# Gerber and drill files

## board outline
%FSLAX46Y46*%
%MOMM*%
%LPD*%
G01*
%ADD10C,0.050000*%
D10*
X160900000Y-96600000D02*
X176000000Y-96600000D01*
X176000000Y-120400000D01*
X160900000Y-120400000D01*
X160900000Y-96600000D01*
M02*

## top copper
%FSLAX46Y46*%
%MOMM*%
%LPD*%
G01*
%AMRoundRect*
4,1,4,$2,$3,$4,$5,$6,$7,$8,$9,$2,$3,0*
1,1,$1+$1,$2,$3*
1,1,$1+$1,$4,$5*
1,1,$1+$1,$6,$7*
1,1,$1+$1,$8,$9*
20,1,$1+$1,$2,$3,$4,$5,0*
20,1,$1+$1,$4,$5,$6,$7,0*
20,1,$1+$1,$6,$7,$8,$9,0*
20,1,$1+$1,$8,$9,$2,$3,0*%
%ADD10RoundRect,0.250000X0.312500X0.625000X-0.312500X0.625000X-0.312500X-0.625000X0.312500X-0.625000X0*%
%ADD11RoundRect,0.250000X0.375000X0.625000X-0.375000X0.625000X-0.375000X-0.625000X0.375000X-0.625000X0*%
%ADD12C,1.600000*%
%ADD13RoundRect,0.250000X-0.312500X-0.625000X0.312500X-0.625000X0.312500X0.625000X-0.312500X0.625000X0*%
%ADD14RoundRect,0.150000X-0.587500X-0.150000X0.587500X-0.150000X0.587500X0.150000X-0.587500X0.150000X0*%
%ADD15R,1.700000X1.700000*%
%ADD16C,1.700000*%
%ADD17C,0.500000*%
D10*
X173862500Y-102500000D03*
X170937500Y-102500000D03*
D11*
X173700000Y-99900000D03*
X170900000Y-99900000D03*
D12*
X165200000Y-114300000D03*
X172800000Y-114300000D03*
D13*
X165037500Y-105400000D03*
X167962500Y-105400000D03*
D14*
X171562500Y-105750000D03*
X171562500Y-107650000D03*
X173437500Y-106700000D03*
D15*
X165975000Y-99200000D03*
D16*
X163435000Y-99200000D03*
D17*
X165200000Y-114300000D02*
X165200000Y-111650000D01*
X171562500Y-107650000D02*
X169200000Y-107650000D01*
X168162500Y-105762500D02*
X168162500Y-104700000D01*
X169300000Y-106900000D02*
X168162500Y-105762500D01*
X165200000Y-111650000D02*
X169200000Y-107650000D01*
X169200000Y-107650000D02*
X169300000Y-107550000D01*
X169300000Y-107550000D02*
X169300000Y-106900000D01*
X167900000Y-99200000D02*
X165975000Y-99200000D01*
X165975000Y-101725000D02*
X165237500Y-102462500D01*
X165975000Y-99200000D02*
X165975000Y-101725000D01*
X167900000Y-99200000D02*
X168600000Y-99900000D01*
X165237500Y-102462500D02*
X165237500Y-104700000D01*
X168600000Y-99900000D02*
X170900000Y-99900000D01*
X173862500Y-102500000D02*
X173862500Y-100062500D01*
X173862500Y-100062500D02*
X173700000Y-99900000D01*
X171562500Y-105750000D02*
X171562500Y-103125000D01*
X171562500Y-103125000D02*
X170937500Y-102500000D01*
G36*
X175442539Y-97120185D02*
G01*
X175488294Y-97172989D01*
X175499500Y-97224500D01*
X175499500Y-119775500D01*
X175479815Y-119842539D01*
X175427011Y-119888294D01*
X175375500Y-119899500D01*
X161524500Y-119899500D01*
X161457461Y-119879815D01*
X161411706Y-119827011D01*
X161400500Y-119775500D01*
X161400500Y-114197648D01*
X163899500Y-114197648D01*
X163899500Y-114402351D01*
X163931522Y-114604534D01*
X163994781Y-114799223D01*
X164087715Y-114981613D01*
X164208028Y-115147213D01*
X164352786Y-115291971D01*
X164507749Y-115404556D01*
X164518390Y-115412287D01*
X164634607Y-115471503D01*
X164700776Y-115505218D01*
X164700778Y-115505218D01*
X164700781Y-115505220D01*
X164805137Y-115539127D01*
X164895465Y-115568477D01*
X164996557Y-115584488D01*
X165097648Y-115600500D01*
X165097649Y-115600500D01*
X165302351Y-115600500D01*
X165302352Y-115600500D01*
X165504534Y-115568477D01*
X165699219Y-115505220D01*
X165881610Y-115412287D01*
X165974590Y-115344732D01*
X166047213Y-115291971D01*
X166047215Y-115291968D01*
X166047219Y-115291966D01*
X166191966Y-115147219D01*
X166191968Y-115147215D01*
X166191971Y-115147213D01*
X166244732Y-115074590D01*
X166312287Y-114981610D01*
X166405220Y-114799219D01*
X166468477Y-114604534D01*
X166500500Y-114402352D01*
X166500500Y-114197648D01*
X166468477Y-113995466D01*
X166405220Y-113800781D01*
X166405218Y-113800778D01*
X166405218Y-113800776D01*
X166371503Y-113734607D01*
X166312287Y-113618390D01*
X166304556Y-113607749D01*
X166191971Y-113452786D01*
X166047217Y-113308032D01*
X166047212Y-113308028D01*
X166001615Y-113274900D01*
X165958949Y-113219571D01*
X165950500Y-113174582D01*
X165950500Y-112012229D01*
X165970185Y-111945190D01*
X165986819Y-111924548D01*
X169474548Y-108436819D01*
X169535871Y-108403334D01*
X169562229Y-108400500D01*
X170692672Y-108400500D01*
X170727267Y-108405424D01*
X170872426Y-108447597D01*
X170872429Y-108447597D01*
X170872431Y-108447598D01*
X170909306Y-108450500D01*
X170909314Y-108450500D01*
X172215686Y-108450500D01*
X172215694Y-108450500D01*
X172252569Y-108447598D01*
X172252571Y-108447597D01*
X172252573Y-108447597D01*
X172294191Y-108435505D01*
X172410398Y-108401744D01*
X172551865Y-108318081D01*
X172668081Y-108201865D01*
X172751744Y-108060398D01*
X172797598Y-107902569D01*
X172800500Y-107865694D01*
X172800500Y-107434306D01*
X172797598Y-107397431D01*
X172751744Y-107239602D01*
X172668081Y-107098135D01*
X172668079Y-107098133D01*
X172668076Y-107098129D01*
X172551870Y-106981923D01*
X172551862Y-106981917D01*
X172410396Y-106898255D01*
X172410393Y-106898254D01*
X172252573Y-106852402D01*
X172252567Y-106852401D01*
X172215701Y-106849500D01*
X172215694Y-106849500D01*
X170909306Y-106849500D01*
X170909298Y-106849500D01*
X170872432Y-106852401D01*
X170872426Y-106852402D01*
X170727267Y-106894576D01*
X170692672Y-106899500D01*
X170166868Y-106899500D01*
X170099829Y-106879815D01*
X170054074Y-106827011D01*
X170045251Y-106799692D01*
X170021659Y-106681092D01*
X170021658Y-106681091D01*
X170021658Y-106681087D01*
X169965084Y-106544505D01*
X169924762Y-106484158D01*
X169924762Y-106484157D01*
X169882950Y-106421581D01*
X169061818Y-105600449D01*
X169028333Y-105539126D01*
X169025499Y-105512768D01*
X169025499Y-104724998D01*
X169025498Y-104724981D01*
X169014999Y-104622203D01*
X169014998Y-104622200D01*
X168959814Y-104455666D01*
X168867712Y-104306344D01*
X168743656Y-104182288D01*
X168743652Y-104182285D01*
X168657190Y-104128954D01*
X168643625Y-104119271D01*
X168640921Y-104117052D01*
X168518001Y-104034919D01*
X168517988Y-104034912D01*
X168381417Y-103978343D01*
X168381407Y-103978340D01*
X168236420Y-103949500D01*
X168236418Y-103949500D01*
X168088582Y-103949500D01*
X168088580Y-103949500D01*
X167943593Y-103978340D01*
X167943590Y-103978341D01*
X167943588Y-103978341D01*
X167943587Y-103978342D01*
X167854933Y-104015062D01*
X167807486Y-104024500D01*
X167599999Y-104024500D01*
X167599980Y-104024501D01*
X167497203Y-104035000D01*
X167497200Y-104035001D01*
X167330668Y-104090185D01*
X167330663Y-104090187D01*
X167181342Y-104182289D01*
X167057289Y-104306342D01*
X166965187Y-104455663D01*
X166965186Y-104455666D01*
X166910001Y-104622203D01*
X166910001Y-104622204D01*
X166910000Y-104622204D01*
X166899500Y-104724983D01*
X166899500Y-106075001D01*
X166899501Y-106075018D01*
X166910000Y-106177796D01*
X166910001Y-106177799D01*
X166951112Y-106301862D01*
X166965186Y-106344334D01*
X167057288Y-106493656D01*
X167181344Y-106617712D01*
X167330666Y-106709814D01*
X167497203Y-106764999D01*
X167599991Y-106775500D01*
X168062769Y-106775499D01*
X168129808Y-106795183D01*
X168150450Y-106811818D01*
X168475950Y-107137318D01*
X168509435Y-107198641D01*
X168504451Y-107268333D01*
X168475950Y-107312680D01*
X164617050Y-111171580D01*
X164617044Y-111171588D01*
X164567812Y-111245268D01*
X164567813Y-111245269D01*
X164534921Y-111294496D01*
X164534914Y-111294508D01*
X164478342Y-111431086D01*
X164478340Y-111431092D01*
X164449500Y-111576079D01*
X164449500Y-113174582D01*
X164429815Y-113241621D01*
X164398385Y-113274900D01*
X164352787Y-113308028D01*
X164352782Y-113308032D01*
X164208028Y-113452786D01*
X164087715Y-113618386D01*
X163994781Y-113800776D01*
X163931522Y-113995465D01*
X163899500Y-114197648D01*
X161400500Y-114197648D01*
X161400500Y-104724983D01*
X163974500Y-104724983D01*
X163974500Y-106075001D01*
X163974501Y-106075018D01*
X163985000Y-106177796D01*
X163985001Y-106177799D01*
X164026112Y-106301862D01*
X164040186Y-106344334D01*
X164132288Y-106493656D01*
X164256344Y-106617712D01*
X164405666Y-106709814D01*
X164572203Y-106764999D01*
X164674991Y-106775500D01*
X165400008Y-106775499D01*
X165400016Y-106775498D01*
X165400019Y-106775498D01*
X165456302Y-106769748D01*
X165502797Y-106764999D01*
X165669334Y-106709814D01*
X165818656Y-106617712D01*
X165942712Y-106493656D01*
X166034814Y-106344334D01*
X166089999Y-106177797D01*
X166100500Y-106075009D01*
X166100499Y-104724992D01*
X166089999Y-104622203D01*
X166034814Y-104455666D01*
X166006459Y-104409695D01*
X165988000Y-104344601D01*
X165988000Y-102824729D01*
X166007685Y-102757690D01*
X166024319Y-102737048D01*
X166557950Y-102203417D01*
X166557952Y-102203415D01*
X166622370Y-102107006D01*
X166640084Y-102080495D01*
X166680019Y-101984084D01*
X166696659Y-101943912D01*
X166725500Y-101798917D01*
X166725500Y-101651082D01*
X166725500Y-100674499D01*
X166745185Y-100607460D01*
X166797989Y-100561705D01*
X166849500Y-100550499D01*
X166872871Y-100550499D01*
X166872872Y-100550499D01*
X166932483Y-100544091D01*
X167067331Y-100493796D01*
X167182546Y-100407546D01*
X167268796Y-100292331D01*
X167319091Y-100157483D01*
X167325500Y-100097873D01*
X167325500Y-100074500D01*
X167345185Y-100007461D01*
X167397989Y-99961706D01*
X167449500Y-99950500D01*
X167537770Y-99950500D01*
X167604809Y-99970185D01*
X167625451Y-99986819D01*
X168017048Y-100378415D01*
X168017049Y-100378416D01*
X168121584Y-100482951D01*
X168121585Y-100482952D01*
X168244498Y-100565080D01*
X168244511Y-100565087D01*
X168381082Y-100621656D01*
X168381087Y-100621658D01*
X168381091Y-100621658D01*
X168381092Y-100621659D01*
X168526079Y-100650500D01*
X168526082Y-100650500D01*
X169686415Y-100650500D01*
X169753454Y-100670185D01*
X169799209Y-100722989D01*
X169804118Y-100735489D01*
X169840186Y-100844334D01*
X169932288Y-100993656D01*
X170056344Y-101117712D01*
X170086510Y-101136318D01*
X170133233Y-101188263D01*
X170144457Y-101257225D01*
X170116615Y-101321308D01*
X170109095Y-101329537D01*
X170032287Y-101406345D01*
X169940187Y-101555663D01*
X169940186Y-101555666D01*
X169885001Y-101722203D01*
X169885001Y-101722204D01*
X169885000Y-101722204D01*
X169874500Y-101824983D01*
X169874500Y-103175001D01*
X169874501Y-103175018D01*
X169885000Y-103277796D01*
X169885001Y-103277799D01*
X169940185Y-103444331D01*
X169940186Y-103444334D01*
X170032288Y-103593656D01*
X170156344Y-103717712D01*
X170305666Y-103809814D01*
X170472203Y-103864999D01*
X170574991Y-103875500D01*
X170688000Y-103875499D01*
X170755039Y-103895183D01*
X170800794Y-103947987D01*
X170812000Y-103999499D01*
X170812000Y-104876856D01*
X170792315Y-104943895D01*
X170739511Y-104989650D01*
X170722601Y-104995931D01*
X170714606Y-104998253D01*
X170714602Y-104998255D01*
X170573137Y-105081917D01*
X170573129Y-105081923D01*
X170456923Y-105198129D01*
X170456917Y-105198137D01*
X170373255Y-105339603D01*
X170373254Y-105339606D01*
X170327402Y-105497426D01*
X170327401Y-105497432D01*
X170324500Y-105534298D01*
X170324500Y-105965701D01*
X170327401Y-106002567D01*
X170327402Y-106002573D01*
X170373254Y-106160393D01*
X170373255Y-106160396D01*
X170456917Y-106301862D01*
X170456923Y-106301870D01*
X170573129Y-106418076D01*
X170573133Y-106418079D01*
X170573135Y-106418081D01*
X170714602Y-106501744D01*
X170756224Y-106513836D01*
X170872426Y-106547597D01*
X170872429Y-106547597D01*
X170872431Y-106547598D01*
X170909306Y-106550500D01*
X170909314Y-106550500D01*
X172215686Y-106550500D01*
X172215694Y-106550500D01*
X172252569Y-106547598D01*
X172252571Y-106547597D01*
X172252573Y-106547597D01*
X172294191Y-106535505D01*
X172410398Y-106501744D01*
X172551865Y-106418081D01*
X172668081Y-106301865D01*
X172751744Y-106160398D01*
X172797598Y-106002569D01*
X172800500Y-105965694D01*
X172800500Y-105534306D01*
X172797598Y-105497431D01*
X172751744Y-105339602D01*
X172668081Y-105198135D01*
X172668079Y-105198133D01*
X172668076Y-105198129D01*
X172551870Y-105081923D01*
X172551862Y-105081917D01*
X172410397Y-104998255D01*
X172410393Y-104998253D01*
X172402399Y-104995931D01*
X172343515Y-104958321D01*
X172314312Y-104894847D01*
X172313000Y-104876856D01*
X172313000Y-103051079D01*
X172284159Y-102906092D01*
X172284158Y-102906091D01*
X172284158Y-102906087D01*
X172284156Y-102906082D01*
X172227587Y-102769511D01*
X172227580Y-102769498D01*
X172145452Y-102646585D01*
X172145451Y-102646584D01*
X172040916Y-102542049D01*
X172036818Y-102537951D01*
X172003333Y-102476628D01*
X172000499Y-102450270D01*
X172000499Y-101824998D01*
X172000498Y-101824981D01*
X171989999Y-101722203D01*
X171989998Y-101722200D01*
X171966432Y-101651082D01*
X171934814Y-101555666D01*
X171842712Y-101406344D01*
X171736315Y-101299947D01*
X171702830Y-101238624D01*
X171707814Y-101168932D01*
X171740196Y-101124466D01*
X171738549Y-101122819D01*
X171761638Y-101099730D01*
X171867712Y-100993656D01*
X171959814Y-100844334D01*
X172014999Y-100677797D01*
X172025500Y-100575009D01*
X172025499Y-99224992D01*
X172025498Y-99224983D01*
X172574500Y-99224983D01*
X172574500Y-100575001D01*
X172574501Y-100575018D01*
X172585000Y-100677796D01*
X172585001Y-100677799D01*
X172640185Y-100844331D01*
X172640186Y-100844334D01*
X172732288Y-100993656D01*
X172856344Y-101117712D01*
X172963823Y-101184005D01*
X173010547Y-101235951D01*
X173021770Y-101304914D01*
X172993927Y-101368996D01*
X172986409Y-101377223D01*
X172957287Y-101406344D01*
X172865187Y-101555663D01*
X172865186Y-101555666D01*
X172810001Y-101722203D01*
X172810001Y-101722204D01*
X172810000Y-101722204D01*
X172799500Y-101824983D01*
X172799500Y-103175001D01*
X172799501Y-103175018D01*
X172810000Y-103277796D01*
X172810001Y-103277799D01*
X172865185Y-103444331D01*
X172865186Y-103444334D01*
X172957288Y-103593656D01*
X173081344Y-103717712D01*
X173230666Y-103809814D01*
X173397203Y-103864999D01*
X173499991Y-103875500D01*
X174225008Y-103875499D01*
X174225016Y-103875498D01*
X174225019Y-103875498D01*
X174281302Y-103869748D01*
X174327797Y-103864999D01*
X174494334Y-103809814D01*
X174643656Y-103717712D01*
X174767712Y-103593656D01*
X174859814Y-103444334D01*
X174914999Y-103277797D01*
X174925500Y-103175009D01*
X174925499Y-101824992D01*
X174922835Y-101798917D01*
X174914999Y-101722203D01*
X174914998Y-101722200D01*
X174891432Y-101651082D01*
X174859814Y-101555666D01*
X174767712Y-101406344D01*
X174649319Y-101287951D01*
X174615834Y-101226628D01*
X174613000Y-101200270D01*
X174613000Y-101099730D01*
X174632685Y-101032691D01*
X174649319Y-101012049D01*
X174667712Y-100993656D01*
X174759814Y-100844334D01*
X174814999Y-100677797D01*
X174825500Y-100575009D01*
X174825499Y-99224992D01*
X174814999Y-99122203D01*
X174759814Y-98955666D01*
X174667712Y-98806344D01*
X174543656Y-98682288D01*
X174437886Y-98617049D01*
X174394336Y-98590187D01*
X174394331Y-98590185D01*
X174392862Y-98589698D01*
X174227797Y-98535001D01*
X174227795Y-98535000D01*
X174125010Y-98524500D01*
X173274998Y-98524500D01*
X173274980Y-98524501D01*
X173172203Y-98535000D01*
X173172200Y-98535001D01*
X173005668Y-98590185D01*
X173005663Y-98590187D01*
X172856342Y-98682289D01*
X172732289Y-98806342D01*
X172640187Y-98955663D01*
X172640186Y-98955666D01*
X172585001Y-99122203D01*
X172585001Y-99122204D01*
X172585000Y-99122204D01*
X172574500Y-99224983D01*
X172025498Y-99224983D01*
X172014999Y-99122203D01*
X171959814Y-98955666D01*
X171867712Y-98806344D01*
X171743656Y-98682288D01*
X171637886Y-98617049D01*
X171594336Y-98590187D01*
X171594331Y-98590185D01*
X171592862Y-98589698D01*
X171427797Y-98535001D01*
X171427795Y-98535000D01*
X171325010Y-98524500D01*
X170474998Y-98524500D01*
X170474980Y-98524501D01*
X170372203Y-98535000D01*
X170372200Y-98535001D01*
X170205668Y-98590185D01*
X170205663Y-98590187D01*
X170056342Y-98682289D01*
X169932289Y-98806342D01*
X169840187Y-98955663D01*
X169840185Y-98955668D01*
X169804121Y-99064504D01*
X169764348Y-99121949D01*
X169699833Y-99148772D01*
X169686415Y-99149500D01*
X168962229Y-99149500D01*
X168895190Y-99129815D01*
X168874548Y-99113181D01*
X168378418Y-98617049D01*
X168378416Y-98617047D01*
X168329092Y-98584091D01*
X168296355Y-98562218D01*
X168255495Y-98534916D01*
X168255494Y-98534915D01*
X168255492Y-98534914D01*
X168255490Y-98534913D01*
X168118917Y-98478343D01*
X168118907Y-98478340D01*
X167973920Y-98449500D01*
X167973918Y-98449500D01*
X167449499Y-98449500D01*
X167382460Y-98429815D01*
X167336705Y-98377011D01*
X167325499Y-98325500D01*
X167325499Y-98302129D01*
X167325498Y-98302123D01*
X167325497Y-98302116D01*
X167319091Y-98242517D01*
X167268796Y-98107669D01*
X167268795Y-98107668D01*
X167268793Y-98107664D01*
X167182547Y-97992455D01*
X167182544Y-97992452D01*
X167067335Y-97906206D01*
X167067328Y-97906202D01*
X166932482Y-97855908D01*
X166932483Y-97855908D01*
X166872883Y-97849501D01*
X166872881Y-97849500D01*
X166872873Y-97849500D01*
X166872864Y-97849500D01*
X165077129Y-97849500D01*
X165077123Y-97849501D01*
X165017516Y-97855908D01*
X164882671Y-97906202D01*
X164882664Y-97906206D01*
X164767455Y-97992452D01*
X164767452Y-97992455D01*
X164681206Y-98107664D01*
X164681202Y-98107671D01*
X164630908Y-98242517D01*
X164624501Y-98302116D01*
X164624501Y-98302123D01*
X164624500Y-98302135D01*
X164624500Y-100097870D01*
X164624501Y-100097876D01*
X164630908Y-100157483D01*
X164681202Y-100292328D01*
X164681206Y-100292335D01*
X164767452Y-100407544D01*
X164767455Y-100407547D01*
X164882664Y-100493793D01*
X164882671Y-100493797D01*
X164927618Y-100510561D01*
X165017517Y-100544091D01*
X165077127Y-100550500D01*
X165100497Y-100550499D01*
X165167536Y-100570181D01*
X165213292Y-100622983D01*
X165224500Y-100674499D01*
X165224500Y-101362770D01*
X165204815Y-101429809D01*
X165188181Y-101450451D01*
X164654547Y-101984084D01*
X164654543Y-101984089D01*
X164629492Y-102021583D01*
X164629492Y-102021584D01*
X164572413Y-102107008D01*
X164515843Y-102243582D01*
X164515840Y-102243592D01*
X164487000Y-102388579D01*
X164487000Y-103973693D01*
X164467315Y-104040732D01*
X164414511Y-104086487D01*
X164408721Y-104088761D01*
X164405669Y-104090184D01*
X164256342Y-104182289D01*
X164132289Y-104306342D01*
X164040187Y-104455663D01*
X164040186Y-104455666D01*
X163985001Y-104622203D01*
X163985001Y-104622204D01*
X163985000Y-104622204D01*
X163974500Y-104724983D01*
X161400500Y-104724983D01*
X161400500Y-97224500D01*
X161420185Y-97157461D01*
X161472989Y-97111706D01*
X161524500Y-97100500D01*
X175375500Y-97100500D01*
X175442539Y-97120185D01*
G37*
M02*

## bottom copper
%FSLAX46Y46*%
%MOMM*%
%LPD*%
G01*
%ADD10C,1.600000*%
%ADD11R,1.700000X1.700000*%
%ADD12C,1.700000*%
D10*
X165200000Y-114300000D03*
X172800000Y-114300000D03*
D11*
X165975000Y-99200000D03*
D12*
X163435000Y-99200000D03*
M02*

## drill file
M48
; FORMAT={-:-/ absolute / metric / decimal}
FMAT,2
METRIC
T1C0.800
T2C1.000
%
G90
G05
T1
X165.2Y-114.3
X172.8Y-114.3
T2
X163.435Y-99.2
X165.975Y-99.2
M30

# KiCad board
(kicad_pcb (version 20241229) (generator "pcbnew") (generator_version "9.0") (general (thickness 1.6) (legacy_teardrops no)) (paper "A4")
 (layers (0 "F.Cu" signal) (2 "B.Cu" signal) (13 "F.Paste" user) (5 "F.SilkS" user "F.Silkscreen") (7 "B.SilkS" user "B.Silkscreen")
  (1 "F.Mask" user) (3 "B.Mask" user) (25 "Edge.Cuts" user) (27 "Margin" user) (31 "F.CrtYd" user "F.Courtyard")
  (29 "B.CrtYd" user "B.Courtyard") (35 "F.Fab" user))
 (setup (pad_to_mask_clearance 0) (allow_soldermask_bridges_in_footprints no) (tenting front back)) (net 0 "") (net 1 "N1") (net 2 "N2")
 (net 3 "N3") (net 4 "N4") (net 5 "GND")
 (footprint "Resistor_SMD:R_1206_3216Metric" (layer "F.Cu") (at 172.4 102.5 180)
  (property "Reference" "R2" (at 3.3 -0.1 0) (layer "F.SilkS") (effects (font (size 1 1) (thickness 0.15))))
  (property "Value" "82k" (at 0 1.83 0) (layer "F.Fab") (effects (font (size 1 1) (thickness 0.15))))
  (pad "1" smd roundrect (at -1.4625 0 180) (size 1.125 1.75) (layers "F.Cu" "F.Mask" "F.Paste") (roundrect_rratio 0.222222) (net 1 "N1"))
  (pad "2" smd roundrect (at 1.4625 0 180) (size 1.125 1.75) (layers "F.Cu" "F.Mask" "F.Paste") (roundrect_rratio 0.222222) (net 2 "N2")))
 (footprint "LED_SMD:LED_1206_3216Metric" (layer "F.Cu") (at 172.3 99.9 180)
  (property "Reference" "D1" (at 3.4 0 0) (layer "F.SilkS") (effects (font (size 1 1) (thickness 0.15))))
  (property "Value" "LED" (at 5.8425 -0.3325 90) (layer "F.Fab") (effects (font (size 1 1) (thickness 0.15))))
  (pad "1" smd roundrect (at -1.4 0 180) (size 1.25 1.75) (layers "F.Cu" "F.Mask" "F.Paste") (roundrect_rratio 0.2) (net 1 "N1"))
  (pad "2" smd roundrect (at 1.4 0 180) (size 1.25 1.75) (layers "F.Cu" "F.Mask" "F.Paste") (roundrect_rratio 0.2) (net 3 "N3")))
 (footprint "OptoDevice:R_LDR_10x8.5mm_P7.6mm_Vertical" (layer "F.Cu") (at 165.2 114.3)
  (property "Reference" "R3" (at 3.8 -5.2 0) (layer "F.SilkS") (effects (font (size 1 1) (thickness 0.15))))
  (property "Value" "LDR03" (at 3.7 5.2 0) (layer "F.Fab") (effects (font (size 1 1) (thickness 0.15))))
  (pad "1" thru_hole circle (at 0 0) (size 1.6 1.6) (drill 0.8) (layers "*.Cu" "*.Mask") (remove_unused_layers no) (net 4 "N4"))
  (pad "2" thru_hole circle (at 7.6 0) (size 1.6 1.6) (drill 0.8) (layers "*.Cu" "*.Mask") (remove_unused_layers no) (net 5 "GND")))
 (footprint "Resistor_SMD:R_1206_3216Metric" (layer "F.Cu") (at 166.5 105.4)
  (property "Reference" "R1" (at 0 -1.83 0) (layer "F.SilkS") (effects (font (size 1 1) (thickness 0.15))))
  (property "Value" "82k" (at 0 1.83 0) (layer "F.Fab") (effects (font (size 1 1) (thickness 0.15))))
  (pad "1" smd roundrect (at -1.4625 0) (size 1.125 1.75) (layers "F.Cu" "F.Mask" "F.Paste") (roundrect_rratio 0.222222) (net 3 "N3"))
  (pad "2" smd roundrect (at 1.4625 0) (size 1.125 1.75) (layers "F.Cu" "F.Mask" "F.Paste") (roundrect_rratio 0.222222) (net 4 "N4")))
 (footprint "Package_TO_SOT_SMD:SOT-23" (layer "F.Cu") (at 172.5 106.7)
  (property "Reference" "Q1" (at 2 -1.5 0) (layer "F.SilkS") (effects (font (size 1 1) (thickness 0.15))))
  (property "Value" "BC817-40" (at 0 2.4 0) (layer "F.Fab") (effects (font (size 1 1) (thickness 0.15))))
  (pad "1" smd roundrect (at -0.9375 -0.95) (size 1.475 0.6) (layers "F.Cu" "F.Mask" "F.Paste") (roundrect_rratio 0.25) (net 2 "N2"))
  (pad "2" smd roundrect (at -0.9375 0.95) (size 1.475 0.6) (layers "F.Cu" "F.Mask" "F.Paste") (roundrect_rratio 0.25) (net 4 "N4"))
  (pad "3" smd roundrect (at 0.9375 0) (size 1.475 0.6) (layers "F.Cu" "F.Mask" "F.Paste") (roundrect_rratio 0.25) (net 5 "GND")))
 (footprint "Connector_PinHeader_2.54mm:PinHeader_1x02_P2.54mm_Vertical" (layer "F.Cu") (at 165.975 99.2 -90)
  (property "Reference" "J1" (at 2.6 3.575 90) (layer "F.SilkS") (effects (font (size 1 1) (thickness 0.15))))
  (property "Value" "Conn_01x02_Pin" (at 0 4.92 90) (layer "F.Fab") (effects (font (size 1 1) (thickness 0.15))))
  (pad "1" thru_hole rect (at 0 0 270) (size 1.7 1.7) (drill 1) (layers "*.Cu" "*.Mask") (remove_unused_layers no) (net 3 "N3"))
  (pad "2" thru_hole circle (at 0 2.54 270) (size 1.7 1.7) (drill 1) (layers "*.Cu" "*.Mask") (remove_unused_layers no) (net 5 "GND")))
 (gr_rect (start 160.9 96.6) (end 176 120.4) (stroke (width 0.05) (type default)) (fill no) (layer "Edge.Cuts"))
 (segment (start 165.2 114.3) (end 165.2 111.65) (width 0.5) (layer "F.Cu") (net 4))
 (segment (start 171.5625 107.65) (end 169.2 107.65) (width 0.5) (layer "F.Cu") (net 4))
 (segment (start 168.1625 105.7625) (end 168.1625 104.7) (width 0.5) (layer "F.Cu") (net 4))
 (segment (start 169.3 106.9) (end 168.1625 105.7625) (width 0.5) (layer "F.Cu") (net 4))
 (segment (start 165.2 111.65) (end 169.2 107.65) (width 0.5) (layer "F.Cu") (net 4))
 (segment (start 169.2 107.65) (end 169.3 107.55) (width 0.5) (layer "F.Cu") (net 4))
 (segment (start 169.3 107.55) (end 169.3 106.9) (width 0.5) (layer "F.Cu") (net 4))
 (segment (start 167.9 99.2) (end 165.975 99.2) (width 0.5) (layer "F.Cu") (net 3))
 (segment (start 165.975 101.725) (end 165.2375 102.4625) (width 0.5) (layer "F.Cu") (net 3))
 (segment (start 165.975 99.2) (end 165.975 101.725) (width 0.5) (layer "F.Cu") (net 3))
 (segment (start 167.9 99.2) (end 168.6 99.9) (width 0.5) (layer "F.Cu") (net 3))
 (segment (start 165.2375 102.4625) (end 165.2375 104.7) (width 0.5) (layer "F.Cu") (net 3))
 (segment (start 168.6 99.9) (end 170.9 99.9) (width 0.5) (layer "F.Cu") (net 3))
 (segment (start 173.8625 102.5) (end 173.8625 100.0625) (width 0.5) (layer "F.Cu") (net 1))
 (segment (start 173.8625 100.0625) (end 173.7 99.9) (width 0.5) (layer "F.Cu") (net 1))
 (segment (start 171.5625 105.75) (end 171.5625 103.125) (width 0.5) (layer "F.Cu") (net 2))
 (segment (start 171.5625 103.125) (end 170.9375 102.5) (width 0.5) (layer "F.Cu") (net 2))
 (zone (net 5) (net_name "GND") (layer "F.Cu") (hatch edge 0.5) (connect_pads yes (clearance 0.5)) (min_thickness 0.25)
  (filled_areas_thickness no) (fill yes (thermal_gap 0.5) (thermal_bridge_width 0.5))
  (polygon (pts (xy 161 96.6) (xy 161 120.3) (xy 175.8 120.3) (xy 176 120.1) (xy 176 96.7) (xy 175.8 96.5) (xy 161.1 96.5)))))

